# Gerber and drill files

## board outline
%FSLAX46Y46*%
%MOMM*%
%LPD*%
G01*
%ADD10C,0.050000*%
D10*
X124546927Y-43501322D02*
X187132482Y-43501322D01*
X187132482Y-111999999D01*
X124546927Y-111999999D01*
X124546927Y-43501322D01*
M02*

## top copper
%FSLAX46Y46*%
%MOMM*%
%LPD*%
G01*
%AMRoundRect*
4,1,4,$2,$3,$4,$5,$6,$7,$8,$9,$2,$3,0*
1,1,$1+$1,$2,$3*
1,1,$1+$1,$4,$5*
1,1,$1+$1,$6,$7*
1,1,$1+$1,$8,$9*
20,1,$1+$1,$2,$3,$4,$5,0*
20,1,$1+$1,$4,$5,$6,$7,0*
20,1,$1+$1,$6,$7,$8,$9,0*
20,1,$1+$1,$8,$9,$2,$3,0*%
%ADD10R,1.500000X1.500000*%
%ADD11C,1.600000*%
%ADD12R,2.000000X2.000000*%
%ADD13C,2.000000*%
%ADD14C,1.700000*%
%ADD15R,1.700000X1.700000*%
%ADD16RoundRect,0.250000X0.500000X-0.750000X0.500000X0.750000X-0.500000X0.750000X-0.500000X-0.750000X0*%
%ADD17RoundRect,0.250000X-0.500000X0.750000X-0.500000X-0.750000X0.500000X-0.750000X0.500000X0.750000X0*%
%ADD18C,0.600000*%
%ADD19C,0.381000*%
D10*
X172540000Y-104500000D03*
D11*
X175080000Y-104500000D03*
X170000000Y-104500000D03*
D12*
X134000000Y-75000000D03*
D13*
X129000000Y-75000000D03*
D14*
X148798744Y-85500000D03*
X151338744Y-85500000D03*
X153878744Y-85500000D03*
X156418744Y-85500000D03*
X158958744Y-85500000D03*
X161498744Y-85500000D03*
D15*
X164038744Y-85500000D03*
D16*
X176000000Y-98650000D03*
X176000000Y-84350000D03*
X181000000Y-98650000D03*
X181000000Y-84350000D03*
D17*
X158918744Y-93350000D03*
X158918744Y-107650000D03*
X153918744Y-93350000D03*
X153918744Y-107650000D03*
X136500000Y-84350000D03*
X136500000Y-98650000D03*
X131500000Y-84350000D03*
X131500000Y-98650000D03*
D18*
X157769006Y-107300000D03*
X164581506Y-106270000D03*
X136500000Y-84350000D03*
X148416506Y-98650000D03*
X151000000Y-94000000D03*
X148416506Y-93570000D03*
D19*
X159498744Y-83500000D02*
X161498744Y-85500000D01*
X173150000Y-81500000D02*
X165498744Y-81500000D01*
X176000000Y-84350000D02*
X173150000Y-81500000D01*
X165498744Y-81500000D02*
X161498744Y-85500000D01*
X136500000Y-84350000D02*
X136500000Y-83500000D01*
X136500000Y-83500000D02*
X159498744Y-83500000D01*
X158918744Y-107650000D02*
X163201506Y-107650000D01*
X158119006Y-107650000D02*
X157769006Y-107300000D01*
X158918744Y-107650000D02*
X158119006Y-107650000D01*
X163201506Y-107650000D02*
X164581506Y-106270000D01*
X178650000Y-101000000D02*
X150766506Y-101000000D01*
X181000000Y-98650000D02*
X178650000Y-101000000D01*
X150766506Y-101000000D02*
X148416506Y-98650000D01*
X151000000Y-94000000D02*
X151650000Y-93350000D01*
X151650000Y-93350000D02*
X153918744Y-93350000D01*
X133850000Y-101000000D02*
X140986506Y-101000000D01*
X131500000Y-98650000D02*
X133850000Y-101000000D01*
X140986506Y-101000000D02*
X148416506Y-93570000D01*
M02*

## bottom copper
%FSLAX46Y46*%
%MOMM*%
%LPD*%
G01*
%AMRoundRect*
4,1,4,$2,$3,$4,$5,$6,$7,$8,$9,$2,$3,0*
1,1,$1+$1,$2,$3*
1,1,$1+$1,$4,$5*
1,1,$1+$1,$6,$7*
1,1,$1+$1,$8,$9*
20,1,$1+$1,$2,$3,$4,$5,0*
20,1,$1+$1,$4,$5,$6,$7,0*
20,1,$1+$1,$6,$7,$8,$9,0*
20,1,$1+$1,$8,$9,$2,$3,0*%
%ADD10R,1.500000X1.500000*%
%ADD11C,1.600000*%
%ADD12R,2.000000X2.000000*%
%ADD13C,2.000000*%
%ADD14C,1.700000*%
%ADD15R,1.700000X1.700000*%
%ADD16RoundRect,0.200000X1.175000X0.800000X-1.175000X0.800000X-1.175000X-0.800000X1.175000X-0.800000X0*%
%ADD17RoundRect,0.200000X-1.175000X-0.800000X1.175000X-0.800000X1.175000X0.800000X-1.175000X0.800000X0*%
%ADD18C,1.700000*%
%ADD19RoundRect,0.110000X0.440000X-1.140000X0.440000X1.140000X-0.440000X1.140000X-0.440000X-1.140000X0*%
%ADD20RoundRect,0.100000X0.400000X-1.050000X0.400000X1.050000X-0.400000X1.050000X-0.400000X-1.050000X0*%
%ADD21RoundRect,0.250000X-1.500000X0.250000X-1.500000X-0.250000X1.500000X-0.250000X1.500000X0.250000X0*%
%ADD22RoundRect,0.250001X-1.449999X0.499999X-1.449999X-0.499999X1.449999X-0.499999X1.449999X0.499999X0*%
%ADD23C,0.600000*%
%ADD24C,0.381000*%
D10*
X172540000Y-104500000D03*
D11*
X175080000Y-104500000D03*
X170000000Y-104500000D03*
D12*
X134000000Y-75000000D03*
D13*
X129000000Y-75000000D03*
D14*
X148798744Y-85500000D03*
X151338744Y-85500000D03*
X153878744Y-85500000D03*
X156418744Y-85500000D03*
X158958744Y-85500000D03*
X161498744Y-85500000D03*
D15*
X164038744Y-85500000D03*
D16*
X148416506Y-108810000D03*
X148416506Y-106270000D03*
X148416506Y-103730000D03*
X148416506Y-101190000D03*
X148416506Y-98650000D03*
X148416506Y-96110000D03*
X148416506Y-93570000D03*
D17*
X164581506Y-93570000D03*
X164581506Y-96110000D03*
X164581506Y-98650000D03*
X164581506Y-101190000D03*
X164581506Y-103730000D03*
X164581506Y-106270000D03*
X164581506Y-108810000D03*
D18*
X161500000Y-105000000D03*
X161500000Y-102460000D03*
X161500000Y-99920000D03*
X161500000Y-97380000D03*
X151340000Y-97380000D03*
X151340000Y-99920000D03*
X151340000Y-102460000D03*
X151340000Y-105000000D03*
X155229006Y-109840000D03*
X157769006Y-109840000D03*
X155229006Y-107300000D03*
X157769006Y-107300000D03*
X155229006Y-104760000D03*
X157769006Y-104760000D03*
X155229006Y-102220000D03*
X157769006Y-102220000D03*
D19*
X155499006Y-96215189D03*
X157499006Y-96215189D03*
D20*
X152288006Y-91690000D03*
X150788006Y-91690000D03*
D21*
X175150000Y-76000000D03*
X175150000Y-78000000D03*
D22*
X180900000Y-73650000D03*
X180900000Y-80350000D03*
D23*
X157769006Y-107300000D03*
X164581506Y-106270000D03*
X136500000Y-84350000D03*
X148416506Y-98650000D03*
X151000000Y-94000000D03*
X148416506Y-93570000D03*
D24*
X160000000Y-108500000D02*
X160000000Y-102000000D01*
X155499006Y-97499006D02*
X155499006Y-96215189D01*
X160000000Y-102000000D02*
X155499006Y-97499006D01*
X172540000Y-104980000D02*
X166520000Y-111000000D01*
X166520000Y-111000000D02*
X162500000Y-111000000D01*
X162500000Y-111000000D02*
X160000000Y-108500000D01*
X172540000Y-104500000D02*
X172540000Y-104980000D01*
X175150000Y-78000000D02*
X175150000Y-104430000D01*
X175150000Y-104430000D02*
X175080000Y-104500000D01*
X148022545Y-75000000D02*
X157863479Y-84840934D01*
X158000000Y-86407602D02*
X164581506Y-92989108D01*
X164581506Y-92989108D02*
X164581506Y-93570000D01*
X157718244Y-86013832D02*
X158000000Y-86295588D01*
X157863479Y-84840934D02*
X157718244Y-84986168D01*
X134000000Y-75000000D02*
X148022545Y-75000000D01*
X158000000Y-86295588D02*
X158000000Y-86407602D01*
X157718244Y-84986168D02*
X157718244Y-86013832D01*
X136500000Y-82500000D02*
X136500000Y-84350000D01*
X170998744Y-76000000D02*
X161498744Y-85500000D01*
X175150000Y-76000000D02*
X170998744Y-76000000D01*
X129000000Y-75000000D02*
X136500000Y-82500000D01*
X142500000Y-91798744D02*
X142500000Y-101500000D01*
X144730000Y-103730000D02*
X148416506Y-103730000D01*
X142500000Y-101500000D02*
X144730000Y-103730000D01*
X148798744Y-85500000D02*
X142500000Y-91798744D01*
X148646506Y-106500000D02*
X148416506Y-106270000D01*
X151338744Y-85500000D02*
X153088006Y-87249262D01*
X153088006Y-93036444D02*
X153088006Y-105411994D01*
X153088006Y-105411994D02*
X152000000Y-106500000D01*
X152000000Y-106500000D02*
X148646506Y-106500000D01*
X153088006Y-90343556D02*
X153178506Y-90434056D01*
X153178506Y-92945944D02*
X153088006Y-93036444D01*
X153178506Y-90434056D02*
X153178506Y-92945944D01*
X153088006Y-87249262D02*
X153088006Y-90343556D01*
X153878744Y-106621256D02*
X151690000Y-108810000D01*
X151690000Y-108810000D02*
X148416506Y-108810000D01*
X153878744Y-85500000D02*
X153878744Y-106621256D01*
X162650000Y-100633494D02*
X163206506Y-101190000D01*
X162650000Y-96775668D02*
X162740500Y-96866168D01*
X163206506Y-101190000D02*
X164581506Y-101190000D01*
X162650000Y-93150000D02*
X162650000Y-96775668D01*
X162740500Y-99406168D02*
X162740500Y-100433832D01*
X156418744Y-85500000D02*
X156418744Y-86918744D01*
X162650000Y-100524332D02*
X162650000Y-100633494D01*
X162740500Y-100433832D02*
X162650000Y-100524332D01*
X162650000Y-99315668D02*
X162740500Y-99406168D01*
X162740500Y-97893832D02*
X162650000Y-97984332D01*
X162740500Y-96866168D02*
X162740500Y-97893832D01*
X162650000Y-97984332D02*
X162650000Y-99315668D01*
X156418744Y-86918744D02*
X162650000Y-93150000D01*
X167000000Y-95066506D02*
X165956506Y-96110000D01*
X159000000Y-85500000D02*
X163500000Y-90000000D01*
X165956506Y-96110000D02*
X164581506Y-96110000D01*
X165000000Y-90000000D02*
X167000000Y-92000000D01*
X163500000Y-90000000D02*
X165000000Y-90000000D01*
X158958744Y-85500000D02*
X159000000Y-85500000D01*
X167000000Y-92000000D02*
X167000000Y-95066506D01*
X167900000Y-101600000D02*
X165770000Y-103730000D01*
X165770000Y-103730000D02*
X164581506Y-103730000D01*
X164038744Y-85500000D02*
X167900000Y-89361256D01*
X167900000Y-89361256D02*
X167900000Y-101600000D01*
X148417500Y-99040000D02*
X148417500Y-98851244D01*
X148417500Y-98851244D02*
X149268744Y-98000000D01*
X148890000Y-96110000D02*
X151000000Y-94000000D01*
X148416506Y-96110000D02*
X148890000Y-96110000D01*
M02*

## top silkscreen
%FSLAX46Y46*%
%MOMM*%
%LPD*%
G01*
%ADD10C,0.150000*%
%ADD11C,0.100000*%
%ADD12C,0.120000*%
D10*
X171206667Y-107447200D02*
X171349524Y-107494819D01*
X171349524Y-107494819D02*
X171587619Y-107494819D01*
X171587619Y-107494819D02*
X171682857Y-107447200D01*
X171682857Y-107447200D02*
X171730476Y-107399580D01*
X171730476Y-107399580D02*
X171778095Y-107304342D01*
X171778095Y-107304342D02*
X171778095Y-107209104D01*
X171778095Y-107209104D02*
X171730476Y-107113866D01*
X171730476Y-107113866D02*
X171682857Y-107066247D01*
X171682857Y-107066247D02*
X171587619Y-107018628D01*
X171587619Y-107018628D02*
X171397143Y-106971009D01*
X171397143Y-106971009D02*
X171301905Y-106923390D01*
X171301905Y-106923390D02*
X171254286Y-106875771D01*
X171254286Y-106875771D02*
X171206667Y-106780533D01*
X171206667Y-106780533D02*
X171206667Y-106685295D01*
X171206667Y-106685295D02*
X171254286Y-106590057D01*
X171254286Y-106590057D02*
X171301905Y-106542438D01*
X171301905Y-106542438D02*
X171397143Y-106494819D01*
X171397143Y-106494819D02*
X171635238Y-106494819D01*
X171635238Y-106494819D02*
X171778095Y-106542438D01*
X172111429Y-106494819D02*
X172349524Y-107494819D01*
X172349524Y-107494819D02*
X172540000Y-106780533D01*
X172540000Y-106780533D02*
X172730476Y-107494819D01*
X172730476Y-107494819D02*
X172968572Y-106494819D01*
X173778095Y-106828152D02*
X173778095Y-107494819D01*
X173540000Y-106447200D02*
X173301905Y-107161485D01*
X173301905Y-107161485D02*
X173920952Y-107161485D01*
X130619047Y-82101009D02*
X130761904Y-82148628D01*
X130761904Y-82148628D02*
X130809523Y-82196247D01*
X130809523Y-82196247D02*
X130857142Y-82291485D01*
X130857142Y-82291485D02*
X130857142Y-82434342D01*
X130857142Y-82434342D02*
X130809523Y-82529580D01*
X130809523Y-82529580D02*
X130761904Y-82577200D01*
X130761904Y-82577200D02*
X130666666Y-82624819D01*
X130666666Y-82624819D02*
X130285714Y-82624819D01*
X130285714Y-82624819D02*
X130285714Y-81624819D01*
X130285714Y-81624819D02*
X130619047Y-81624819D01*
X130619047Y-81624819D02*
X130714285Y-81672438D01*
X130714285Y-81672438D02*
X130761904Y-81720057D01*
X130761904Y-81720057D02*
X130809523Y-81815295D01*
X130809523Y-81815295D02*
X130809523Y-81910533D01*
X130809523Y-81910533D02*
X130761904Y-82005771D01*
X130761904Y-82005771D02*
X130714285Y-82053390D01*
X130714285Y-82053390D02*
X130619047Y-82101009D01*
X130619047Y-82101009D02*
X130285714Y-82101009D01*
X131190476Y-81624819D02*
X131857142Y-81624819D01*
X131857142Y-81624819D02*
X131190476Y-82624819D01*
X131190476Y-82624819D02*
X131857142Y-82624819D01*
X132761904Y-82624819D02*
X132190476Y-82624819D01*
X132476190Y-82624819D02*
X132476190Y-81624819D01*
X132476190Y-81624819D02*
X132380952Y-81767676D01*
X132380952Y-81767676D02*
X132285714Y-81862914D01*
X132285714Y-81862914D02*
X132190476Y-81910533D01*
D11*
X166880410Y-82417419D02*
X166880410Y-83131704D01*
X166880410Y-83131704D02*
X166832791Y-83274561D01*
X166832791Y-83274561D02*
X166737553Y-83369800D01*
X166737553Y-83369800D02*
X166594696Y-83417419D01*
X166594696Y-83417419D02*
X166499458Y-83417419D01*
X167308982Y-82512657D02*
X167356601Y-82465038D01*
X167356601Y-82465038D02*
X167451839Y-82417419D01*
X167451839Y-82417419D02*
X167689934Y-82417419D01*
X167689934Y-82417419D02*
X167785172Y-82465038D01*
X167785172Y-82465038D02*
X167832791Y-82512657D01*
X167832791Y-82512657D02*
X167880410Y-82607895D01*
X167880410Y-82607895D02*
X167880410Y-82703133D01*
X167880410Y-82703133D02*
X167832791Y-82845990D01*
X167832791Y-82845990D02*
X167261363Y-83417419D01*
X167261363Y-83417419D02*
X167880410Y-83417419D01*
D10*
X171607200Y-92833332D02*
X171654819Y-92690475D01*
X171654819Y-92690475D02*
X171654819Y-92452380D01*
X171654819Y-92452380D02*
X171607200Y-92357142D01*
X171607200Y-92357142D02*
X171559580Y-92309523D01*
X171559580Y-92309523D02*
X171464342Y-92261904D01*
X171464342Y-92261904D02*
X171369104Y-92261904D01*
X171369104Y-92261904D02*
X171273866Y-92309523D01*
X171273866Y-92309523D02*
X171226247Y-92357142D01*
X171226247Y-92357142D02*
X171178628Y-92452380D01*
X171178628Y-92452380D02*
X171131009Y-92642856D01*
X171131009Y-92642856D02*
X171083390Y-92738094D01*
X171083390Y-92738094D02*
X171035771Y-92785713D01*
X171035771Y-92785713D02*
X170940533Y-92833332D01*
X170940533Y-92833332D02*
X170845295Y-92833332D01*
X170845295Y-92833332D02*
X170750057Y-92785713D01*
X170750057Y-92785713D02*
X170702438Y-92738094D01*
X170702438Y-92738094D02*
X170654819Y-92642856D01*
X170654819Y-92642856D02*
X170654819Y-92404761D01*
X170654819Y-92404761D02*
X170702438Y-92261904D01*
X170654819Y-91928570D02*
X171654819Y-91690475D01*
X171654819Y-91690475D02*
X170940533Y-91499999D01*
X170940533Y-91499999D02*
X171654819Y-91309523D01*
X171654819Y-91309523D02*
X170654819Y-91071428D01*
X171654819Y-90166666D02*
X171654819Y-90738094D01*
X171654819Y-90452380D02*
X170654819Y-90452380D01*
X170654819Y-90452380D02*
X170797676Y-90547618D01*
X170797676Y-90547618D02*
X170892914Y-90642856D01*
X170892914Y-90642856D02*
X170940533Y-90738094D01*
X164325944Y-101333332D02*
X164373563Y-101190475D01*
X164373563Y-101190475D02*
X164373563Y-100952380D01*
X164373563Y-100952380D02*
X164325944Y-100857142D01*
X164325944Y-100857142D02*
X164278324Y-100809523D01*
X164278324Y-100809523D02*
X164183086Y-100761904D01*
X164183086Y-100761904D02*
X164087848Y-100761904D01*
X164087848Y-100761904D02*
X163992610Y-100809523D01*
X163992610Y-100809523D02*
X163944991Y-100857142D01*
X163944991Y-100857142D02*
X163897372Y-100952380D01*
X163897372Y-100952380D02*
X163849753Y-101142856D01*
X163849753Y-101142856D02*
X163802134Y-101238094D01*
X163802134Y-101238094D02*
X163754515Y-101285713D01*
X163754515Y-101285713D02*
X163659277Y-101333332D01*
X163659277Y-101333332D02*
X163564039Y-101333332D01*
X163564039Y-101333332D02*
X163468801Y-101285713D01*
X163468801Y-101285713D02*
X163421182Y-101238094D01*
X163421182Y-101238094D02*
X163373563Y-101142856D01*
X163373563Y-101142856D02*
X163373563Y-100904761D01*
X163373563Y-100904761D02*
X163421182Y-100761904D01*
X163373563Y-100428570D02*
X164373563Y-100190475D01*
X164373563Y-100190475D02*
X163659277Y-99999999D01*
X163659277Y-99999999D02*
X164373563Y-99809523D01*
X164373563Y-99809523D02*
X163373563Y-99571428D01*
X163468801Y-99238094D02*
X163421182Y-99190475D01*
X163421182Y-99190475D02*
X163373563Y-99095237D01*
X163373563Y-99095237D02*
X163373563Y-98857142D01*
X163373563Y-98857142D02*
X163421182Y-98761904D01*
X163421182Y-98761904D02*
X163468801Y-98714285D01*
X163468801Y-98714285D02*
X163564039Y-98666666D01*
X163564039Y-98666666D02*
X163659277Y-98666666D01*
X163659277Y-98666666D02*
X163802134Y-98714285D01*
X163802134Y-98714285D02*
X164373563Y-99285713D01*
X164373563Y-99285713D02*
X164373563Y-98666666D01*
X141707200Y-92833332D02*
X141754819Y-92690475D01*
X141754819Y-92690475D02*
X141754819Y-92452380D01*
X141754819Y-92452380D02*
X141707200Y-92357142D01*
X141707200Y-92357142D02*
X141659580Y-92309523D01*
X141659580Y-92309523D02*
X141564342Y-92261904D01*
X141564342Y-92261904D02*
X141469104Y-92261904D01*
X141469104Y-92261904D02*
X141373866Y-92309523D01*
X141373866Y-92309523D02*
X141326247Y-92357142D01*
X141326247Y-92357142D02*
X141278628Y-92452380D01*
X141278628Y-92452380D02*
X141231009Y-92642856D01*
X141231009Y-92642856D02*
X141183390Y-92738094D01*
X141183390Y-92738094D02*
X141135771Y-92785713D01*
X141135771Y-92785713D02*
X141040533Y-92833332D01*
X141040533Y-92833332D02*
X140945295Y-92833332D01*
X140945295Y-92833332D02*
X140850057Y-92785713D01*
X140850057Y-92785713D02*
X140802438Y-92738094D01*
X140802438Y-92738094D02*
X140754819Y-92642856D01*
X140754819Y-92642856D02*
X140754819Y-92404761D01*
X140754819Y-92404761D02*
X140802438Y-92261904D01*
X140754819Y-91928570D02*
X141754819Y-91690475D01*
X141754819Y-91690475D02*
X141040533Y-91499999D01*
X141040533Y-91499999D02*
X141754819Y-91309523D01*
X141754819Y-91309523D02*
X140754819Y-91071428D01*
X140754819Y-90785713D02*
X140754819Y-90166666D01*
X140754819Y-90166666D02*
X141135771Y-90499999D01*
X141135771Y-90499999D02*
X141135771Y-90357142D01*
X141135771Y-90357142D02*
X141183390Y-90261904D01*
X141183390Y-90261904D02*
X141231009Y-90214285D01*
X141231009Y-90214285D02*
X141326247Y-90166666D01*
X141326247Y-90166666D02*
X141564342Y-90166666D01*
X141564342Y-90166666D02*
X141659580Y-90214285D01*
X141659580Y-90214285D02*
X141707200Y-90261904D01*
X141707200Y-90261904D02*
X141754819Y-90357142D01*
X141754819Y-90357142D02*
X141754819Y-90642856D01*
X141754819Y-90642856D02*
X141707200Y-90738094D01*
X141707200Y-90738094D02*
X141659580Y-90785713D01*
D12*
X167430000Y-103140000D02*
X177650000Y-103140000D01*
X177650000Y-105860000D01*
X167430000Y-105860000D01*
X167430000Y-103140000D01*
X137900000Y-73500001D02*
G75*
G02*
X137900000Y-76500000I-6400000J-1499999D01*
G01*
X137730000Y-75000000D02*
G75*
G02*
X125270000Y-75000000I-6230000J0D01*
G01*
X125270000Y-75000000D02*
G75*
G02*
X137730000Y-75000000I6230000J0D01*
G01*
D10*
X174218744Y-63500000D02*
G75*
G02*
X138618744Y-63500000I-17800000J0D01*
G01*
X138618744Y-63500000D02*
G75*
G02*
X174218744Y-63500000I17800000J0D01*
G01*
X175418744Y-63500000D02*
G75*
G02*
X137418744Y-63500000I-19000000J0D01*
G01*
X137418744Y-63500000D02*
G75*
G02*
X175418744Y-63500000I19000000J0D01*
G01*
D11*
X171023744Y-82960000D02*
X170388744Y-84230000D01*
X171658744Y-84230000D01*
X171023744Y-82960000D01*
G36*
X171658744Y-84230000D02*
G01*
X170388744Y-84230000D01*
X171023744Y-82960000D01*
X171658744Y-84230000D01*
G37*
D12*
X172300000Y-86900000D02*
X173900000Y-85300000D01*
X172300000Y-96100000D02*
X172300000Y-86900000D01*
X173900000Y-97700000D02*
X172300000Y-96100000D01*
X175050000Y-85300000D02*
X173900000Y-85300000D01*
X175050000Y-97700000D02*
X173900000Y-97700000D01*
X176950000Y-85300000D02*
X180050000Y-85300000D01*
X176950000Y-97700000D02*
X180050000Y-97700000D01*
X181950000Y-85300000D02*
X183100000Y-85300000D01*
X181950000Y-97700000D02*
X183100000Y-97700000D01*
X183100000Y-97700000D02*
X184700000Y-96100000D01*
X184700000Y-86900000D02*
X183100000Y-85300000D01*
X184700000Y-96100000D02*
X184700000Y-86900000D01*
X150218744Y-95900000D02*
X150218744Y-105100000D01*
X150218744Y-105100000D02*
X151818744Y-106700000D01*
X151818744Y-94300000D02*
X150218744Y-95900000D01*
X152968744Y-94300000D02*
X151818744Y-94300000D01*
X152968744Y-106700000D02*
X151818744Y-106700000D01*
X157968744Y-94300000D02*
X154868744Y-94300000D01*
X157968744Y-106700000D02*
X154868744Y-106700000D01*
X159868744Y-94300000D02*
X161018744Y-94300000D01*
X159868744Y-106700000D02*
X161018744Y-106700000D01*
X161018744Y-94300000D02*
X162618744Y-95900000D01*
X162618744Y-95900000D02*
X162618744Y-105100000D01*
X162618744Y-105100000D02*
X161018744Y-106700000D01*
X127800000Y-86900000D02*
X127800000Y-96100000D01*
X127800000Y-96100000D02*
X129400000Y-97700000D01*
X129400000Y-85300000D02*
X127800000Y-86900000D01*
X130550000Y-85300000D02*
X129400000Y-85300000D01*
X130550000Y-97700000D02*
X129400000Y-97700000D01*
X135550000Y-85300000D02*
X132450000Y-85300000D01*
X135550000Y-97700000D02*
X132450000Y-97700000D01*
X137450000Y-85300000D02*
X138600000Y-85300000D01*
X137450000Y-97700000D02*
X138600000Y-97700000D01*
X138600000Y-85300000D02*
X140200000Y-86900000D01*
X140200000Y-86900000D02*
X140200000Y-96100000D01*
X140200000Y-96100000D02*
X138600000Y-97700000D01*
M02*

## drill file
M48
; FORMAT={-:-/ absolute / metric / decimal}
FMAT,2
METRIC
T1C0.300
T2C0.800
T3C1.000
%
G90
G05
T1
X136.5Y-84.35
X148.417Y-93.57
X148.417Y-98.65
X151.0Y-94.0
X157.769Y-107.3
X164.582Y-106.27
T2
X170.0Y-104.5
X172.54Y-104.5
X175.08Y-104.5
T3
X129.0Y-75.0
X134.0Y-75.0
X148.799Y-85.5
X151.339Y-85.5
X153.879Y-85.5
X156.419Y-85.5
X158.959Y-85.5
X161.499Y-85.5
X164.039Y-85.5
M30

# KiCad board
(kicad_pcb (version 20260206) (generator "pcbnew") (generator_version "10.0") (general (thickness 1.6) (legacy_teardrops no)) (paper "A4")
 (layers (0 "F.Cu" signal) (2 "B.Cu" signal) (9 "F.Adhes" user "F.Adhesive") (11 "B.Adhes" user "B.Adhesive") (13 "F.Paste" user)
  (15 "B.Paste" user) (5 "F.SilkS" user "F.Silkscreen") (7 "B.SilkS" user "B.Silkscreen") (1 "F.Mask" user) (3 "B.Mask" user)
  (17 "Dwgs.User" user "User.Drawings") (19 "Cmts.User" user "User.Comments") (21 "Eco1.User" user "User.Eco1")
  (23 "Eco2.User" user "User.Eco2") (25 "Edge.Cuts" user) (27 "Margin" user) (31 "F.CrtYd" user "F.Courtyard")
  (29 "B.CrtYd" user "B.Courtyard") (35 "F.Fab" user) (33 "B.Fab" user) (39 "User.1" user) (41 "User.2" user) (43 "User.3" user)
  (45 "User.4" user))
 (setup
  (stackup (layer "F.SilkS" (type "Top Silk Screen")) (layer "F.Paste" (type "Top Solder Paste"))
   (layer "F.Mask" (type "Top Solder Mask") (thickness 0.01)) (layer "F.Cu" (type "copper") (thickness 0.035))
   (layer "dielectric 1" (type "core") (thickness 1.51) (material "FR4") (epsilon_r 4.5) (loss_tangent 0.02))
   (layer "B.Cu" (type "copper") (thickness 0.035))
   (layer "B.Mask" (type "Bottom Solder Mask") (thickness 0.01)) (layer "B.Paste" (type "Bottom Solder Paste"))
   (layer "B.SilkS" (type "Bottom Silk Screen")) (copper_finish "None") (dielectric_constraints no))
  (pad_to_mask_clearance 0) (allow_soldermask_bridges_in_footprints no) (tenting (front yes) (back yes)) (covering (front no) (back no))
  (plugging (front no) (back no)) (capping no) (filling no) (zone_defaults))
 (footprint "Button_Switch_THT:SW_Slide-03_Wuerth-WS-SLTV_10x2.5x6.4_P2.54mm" (layer "F.Cu") (at 172.54 104.5 180)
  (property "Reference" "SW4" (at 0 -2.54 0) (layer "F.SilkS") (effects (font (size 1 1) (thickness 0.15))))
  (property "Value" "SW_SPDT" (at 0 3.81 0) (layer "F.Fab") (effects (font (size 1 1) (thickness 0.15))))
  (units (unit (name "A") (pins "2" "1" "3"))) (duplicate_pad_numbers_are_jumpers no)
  (fp_rect (start -5.11 -1.36) (end 5.11 1.36) (stroke (width 0.12) (type default)) (fill no) (layer "F.SilkS"))
  (pad "1" thru_hole rect (at 0 0 180) (size 1.5 1.5) (drill 0.8) (layers "*.Cu" "*.Mask") (remove_unused_layers no) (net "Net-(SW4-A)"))
  (pad "2" thru_hole circle (at -2.54 0 180) (size 1.6 1.6) (drill 0.8) (layers "*.Cu" "*.Mask") (remove_unused_layers no)
   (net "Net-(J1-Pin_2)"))
  (pad "3" thru_hole circle (at 2.54 0 180) (size 1.6 1.6) (drill 0.8) (layers "*.Cu" "*.Mask") (remove_unused_layers no)
   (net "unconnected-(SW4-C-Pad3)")))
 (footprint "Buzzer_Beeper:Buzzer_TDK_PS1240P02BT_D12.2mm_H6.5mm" (layer "F.Cu") (at 134 75 180)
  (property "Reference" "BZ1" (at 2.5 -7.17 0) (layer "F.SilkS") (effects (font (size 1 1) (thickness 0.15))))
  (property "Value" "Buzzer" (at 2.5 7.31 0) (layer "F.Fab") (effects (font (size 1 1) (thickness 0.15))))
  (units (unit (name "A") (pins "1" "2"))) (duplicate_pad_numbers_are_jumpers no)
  (fp_arc (start -3.9 1.499999) (mid -4.073431 0) (end -3.9 -1.5) (stroke (width 0.12) (type solid)) (layer "F.SilkS"))
  (fp_circle (center 2.5 0) (end 8.73 0) (stroke (width 0.12) (type solid)) (fill no) (layer "F.SilkS"))
  (pad "1" thru_hole rect (at 0 0 180) (size 2 2) (drill 1) (layers "*.Cu" "*.Mask") (remove_unused_layers no) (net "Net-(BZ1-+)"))
  (pad "2" thru_hole circle (at 5 0 180) (size 2 2) (drill 1) (layers "*.Cu" "*.Mask") (remove_unused_layers no) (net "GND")))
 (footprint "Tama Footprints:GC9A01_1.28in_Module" (layer "F.Cu") (at 164.038744 85.5)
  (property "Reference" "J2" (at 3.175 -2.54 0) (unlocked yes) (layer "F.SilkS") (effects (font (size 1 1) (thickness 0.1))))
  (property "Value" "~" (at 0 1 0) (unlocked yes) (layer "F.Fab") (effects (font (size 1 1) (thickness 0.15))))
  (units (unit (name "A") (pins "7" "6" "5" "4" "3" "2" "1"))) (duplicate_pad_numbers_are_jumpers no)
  (fp_circle (center -7.62 -22) (end 10.18 -22) (stroke (width 0.15) (type solid)) (fill no) (layer "F.SilkS"))
  (fp_circle (center -7.62 -22) (end 11.38 -22) (stroke (width 0.15) (type solid)) (fill no) (layer "F.SilkS"))
  (fp_poly (pts (xy 6.985 -2.54) (xy 6.35 -1.27) (xy 7.62 -1.27)) (stroke (width 0.1) (type solid)) (fill yes) (layer "F.SilkS"))
  (pad "1" thru_hole circle (at -15.24 0) (size 1.7 1.7) (drill 1) (layers "*.Cu" "*.Mask") (remove_unused_layers no) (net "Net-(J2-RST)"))
  (pad "2" thru_hole circle (at -12.7 0) (size 1.7 1.7) (drill 1) (layers "*.Cu" "*.Mask") (remove_unused_layers no) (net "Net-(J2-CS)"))
  (pad "3" thru_hole circle (at -10.16 0) (size 1.7 1.7) (drill 1) (layers "*.Cu" "*.Mask") (remove_unused_layers no) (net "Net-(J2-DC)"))
  (pad "4" thru_hole circle (at -7.62 0) (size 1.7 1.7) (drill 1) (layers "*.Cu" "*.Mask") (remove_unused_layers no) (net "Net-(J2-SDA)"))
  (pad "5" thru_hole circle (at -5.08 0) (size 1.7 1.7) (drill 1) (layers "*.Cu" "*.Mask") (remove_unused_layers no) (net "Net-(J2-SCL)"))
  (pad "6" thru_hole circle (at -2.54 0) (size 1.7 1.7) (drill 1) (layers "*.Cu" "*.Mask") (remove_unused_layers no) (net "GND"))
  (pad "7" thru_hole rect (at 0 0) (size 1.7 1.7) (drill 1) (layers "*.Cu" "*.Mask") (remove_unused_layers no) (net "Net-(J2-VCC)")))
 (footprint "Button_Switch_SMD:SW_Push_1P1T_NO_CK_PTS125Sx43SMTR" (layer "F.Cu") (at 178.5 91.5 90)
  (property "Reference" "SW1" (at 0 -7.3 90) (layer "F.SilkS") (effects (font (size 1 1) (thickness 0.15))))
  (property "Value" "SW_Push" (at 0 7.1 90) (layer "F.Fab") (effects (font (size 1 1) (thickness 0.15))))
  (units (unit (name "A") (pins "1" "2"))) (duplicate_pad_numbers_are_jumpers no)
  (fp_line (start 4.6 -6.2) (end 6.2 -4.6) (stroke (width 0.12) (type solid)) (layer "F.SilkS"))
  (fp_line (start -4.6 -6.2) (end 4.6 -6.2) (stroke (width 0.12) (type solid)) (layer "F.SilkS"))
  (fp_line (start -6.2 -4.6) (end -4.6 -6.2) (stroke (width 0.12) (type solid)) (layer "F.SilkS"))
  (fp_line (start 6.2 -3.45) (end 6.2 -4.6) (stroke (width 0.12) (type solid)) (layer "F.SilkS"))
  (fp_line (start -6.2 -3.45) (end -6.2 -4.6) (stroke (width 0.12) (type solid)) (layer "F.SilkS"))
  (fp_line (start 6.2 -1.55) (end 6.2 1.55) (stroke (width 0.12) (type solid)) (layer "F.SilkS"))
  (fp_line (start -6.2 -1.55) (end -6.2 1.55) (stroke (width 0.12) (type solid)) (layer "F.SilkS"))
  (fp_line (start 6.2 3.45) (end 6.2 4.6) (stroke (width 0.12) (type solid)) (layer "F.SilkS"))
  (fp_line (start -6.2 3.45) (end -6.2 4.6) (stroke (width 0.12) (type solid)) (layer "F.SilkS"))
  (fp_line (start -6.2 4.6) (end -4.6 6.2) (stroke (width 0.12) (type solid)) (layer "F.SilkS"))
  (fp_line (start 4.6 6.2) (end 6.2 4.6) (stroke (width 0.12) (type solid)) (layer "F.SilkS"))
  (fp_line (start -4.6 6.2) (end 4.6 6.2) (stroke (width 0.12) (type solid)) (layer "F.SilkS"))
  (pad "1" smd roundrect (at -7.15 -2.5 90) (size 2 1.5) (layers "F.Cu" "F.Mask" "F.Paste") (roundrect_rratio 0.1666666667))
  (pad "1" smd roundrect (at 7.15 -2.5 90) (size 2 1.5) (layers "F.Cu" "F.Mask" "F.Paste") (roundrect_rratio 0.1666666667) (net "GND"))
  (pad "2" smd roundrect (at -7.15 2.5 90) (size 2 1.5) (layers "F.Cu" "F.Mask" "F.Paste") (roundrect_rratio 0.1666666667)
   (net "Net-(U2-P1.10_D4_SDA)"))
  (pad "2" smd roundrect (at 7.15 2.5 90) (size 2 1.5) (layers "F.Cu" "F.Mask" "F.Paste") (roundrect_rratio 0.1666666667)))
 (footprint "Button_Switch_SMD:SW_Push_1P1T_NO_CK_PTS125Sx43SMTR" (layer "F.Cu") (at 156.418744 100.5 -90)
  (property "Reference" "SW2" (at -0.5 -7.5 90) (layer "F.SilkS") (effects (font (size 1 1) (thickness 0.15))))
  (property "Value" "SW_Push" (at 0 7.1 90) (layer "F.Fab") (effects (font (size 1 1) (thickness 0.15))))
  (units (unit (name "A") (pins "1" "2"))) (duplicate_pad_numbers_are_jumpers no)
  (fp_line (start -4.6 6.2) (end 4.6 6.2) (stroke (width 0.12) (type solid)) (layer "F.SilkS"))
  (fp_line (start 4.6 6.2) (end 6.2 4.6) (stroke (width 0.12) (type solid)) (layer "F.SilkS"))
  (fp_line (start -6.2 4.6) (end -4.6 6.2) (stroke (width 0.12) (type solid)) (layer "F.SilkS"))
  (fp_line (start -6.2 3.45) (end -6.2 4.6) (stroke (width 0.12) (type solid)) (layer "F.SilkS"))
  (fp_line (start 6.2 3.45) (end 6.2 4.6) (stroke (width 0.12) (type solid)) (layer "F.SilkS"))
  (fp_line (start -6.2 -1.55) (end -6.2 1.55) (stroke (width 0.12) (type solid)) (layer "F.SilkS"))
  (fp_line (start 6.2 -1.55) (end 6.2 1.55) (stroke (width 0.12) (type solid)) (layer "F.SilkS"))
  (fp_line (start -6.2 -3.45) (end -6.2 -4.6) (stroke (width 0.12) (type solid)) (layer "F.SilkS"))
  (fp_line (start 6.2 -3.45) (end 6.2 -4.6) (stroke (width 0.12) (type solid)) (layer "F.SilkS"))
  (fp_line (start -6.2 -4.6) (end -4.6 -6.2) (stroke (width 0.12) (type solid)) (layer "F.SilkS"))
  (fp_line (start -4.6 -6.2) (end 4.6 -6.2) (stroke (width 0.12) (type solid)) (layer "F.SilkS"))
  (fp_line (start 4.6 -6.2) (end 6.2 -4.6) (stroke (width 0.12) (type solid)) (layer "F.SilkS"))
  (pad "1" smd roundrect (at -7.15 -2.5 270) (size 2 1.5) (layers "F.Cu" "F.Mask" "F.Paste") (roundrect_rratio 0.1666666667))
  (pad "1" smd roundrect (at 7.15 -2.5 270) (size 2 1.5) (layers "F.Cu" "F.Mask" "F.Paste") (roundrect_rratio 0.1666666667) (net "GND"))
  (pad "2" smd roundrect (at -7.15 2.5 270) (size 2 1.5) (layers "F.Cu" "F.Mask" "F.Paste") (roundrect_rratio 0.1666666667)
   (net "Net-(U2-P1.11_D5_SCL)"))
  (pad "2" smd roundrect (at 7.15 2.5 270) (size 2 1.5) (layers "F.Cu" "F.Mask" "F.Paste") (roundrect_rratio 0.1666666667)))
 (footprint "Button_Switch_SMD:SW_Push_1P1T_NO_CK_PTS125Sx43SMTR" (layer "F.Cu") (at 134 91.5 -90)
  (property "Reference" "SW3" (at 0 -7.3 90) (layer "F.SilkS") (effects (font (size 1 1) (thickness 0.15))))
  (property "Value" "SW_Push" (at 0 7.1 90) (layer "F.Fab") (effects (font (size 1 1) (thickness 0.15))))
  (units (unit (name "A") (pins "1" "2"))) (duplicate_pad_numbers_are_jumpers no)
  (fp_line (start -4.6 6.2) (end 4.6 6.2) (stroke (width 0.12) (type solid)) (layer "F.SilkS"))
  (fp_line (start 4.6 6.2) (end 6.2 4.6) (stroke (width 0.12) (type solid)) (layer "F.SilkS"))
  (fp_line (start -6.2 4.6) (end -4.6 6.2) (stroke (width 0.12) (type solid)) (layer "F.SilkS"))
  (fp_line (start -6.2 3.45) (end -6.2 4.6) (stroke (width 0.12) (type solid)) (layer "F.SilkS"))
  (fp_line (start 6.2 3.45) (end 6.2 4.6) (stroke (width 0.12) (type solid)) (layer "F.SilkS"))
  (fp_line (start -6.2 -1.55) (end -6.2 1.55) (stroke (width 0.12) (type solid)) (layer "F.SilkS"))
  (fp_line (start 6.2 -1.55) (end 6.2 1.55) (stroke (width 0.12) (type solid)) (layer "F.SilkS"))
  (fp_line (start -6.2 -3.45) (end -6.2 -4.6) (stroke (width 0.12) (type solid)) (layer "F.SilkS"))
  (fp_line (start 6.2 -3.45) (end 6.2 -4.6) (stroke (width 0.12) (type solid)) (layer "F.SilkS"))
  (fp_line (start -6.2 -4.6) (end -4.6 -6.2) (stroke (width 0.12) (type solid)) (layer "F.SilkS"))
  (fp_line (start -4.6 -6.2) (end 4.6 -6.2) (stroke (width 0.12) (type solid)) (layer "F.SilkS"))
  (fp_line (start 4.6 -6.2) (end 6.2 -4.6) (stroke (width 0.12) (type solid)) (layer "F.SilkS"))
  (pad "1" smd roundrect (at -7.15 -2.5 270) (size 2 1.5) (layers "F.Cu" "F.Mask" "F.Paste") (roundrect_rratio 0.1666666667) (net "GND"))
  (pad "1" smd roundrect (at 7.15 -2.5 270) (size 2 1.5) (layers "F.Cu" "F.Mask" "F.Paste") (roundrect_rratio 0.1666666667))
  (pad "2" smd roundrect (at -7.15 2.5 270) (size 2 1.5) (layers "F.Cu" "F.Mask" "F.Paste") (roundrect_rratio 0.1666666667))
  (pad "2" smd roundrect (at 7.15 2.5 270) (size 2 1.5) (layers "F.Cu" "F.Mask" "F.Paste") (roundrect_rratio 0.1666666667)
   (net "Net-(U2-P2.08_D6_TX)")))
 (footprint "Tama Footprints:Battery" (layer "B.Cu") (at 156.418744 64.5 -90)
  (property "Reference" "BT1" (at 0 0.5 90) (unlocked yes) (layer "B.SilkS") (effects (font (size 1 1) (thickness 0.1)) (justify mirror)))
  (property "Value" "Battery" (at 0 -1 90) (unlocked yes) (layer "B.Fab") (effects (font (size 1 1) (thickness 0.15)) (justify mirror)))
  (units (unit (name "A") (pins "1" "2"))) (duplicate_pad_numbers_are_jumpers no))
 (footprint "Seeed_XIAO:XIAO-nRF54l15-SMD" (layer "B.Cu") (at 156.499006 101.19 -90)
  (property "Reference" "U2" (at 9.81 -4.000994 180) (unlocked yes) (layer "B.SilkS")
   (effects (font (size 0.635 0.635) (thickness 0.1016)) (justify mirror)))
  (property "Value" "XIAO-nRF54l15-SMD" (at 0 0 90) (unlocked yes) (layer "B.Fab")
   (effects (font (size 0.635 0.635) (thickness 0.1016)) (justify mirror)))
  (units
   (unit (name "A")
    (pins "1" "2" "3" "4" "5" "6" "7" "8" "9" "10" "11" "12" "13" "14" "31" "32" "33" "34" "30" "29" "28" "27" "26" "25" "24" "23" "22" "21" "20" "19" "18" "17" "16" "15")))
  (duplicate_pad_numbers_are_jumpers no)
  (pad "1" smd roundrect (at 7.62 8.0825 180) (size 2.75 2) (layers "B.Cu" "B.Mask" "B.Paste") (roundrect_rratio 0.1) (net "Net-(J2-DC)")
   (thermal_bridge_angle 45))
  (pad "2" smd roundrect (at 5.08 8.0825 180) (size 2.75 2) (layers "B.Cu" "B.Mask" "B.Paste") (roundrect_rratio 0.1) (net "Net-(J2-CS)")
   (thermal_bridge_angle 45))
  (pad "3" smd roundrect (at 2.54 8.0825 180) (size 2.75 2) (layers "B.Cu" "B.Mask" "B.Paste") (roundrect_rratio 0.1) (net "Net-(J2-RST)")
   (thermal_bridge_angle 45))
  (pad "4" smd roundrect (at 0 8.0825 180) (size 2.75 2) (layers "B.Cu" "B.Mask" "B.Paste") (roundrect_rratio 0.1)
   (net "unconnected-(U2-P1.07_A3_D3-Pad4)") (thermal_bridge_angle 45))
  (pad "5" smd roundrect (at -2.54 8.0825 180) (size 2.75 2) (layers "B.Cu" "B.Mask" "B.Paste") (roundrect_rratio 0.1)
   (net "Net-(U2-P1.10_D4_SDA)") (thermal_bridge_angle 45))
  (pad "6" smd roundrect (at -5.08 8.0825 180) (size 2.75 2) (layers "B.Cu" "B.Mask" "B.Paste") (roundrect_rratio 0.1)
   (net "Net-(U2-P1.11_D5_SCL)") (thermal_bridge_angle 45))
  (pad "7" smd roundrect (at -7.62 8.0825 180) (size 2.75 2) (layers "B.Cu" "B.Mask" "B.Paste") (roundrect_rratio 0.1)
   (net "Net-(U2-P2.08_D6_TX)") (thermal_bridge_angle 45))
  (pad "8" smd roundrect (at -7.62 -8.0825) (size 2.75 2) (layers "B.Cu" "B.Mask" "B.Paste") (roundrect_rratio 0.1) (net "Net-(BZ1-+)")
   (thermal_bridge_angle 45))
  (pad "9" smd roundrect (at -5.08 -8.0825) (size 2.75 2) (layers "B.Cu" "B.Mask" "B.Paste") (roundrect_rratio 0.1) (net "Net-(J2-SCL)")
   (thermal_bridge_angle 45))
  (pad "10" smd roundrect (at -2.54 -8.0825) (size 2.75 2) (layers "B.Cu" "B.Mask" "B.Paste") (roundrect_rratio 0.1)
   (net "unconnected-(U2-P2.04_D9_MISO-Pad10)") (thermal_bridge_angle 45))
  (pad "11" smd roundrect (at 0 -8.0825) (size 2.75 2) (layers "B.Cu" "B.Mask" "B.Paste") (roundrect_rratio 0.1) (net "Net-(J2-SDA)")
   (thermal_bridge_angle 45))
  (pad "12" smd roundrect (at 2.54 -8.0825) (size 2.75 2) (layers "B.Cu" "B.Mask" "B.Paste") (roundrect_rratio 0.1) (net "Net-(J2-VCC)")
   (thermal_bridge_angle 45))
  (pad "13" smd roundrect (at 5.08 -8.0825) (size 2.75 2) (layers "B.Cu" "B.Mask" "B.Paste") (roundrect_rratio 0.1) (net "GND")
   (thermal_bridge_angle 45))
  (pad "14" smd roundrect (at 7.62 -8.0825) (size 2.75 2) (layers "B.Cu" "B.Mask" "B.Paste") (roundrect_rratio 0.1)
   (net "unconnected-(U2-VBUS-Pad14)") (thermal_bridge_angle 45))
  (pad "15" smd circle (at 3.81 -5.000994 180) (size 1.7 1.7) (layers "B.Cu" "B.Mask" "B.Paste")
   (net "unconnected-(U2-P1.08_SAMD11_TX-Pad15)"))
  (pad "16" smd circle (at 1.27 -5.000994 180) (size 1.7 1.7) (layers "B.Cu" "B.Mask" "B.Paste")
   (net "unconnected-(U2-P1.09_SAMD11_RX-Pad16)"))
  (pad "17" smd circle (at -1.27 -5.000994 180) (size 1.7 1.7) (layers "B.Cu" "B.Mask" "B.Paste") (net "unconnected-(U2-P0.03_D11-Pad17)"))
  (pad "18" smd circle (at -3.81 -5.000994 180) (size 1.7 1.7) (layers "B.Cu" "B.Mask" "B.Paste") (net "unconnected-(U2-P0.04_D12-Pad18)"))
  (pad "19" smd circle (at -3.81 5.159006 180) (size 1.7 1.7) (layers "B.Cu" "B.Mask" "B.Paste") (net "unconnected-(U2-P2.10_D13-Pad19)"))
  (pad "20" smd circle (at -1.27 5.159006 180) (size 1.7 1.7) (layers "B.Cu" "B.Mask" "B.Paste") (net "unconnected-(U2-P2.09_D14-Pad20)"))
  (pad "21" smd circle (at 1.27 5.159006 180) (size 1.7 1.7) (layers "B.Cu" "B.Mask" "B.Paste") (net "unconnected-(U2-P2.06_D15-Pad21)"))
  (pad "22" smd circle (at 3.81 5.159006 180) (size 1.7 1.7) (layers "B.Cu" "B.Mask" "B.Paste") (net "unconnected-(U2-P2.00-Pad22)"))
  (pad "23" smd circle (at 8.65 1.27 180) (size 1.7 1.7) (layers "B.Cu" "B.Mask" "B.Paste") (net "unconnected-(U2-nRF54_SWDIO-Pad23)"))
  (pad "24" smd circle (at 8.65 -1.27 180) (size 1.7 1.7) (layers "B.Cu" "B.Mask" "B.Paste") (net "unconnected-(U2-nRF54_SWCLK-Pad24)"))
  (pad "25" smd circle (at 6.11 1.27 180) (size 1.7 1.7) (layers "B.Cu" "B.Mask" "B.Paste") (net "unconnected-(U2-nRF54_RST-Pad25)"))
  (pad "26" smd circle (at 6.11 -1.27 180) (size 1.7 1.7) (layers "B.Cu" "B.Mask" "B.Paste") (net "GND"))
  (pad "27" smd circle (at 3.57 1.27 180) (size 1.7 1.7) (layers "B.Cu" "B.Mask" "B.Paste") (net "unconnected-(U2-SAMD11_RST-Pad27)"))
  (pad "28" smd circle (at 3.57 -1.27 180) (size 1.7 1.7) (layers "B.Cu" "B.Mask" "B.Paste") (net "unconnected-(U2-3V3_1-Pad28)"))
  (pad "29" smd circle (at 1.03 1.27 180) (size 1.7 1.7) (layers "B.Cu" "B.Mask" "B.Paste") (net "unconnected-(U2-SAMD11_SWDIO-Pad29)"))
  (pad "30" smd circle (at 1.03 -1.27 180) (size 1.7 1.7) (layers "B.Cu" "B.Mask" "B.Paste") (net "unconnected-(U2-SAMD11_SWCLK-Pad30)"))
  (pad "31" smd roundrect (at -4.974811 1 90) (size 2.5 1.1) (layers "B.Cu" "B.Mask" "B.Paste") (roundrect_rratio 0.1) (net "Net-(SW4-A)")
   (thermal_bridge_angle 45))
  (pad "32" smd roundrect (at -4.974811 -1 90) (size 2.5 1.1) (layers "B.Cu" "B.Mask" "B.Paste") (roundrect_rratio 0.1)
   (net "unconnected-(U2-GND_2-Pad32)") (thermal_bridge_angle 45))
  (pad "33" smd roundrect (at -9.5 4.211 90) (size 2.3 1) (layers "B.Cu" "B.Mask" "B.Paste") (roundrect_rratio 0.1)
   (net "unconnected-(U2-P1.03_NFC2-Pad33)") (thermal_bridge_angle 45))
  (pad "34" smd roundrect (at -9.5 5.711 90) (size 2.3 1) (layers "B.Cu" "B.Mask" "B.Paste") (roundrect_rratio 0.1)
   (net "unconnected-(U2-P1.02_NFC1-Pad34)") (thermal_bridge_angle 45)))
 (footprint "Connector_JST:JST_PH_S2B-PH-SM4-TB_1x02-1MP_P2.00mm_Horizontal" (layer "B.Cu") (at 178 77 -90)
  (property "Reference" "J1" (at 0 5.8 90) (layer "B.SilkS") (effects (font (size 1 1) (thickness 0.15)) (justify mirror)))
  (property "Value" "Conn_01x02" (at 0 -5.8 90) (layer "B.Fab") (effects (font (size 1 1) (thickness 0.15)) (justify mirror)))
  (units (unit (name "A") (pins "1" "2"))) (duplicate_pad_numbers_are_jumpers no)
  (pad "1" smd roundrect (at -1 2.85 270) (size 1 3.5) (layers "B.Cu" "B.Mask" "B.Paste") (roundrect_rratio 0.25) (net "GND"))
  (pad "2" smd roundrect (at 1 2.85 270) (size 1 3.5) (layers "B.Cu" "B.Mask" "B.Paste") (roundrect_rratio 0.25) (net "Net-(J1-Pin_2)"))
  (pad "MP" smd roundrect (at -3.35 -2.9 270) (size 1.5 3.4) (layers "B.Cu" "B.Mask" "B.Paste") (roundrect_rratio 0.166667))
  (pad "MP" smd roundrect (at 3.35 -2.9 270) (size 1.5 3.4) (layers "B.Cu" "B.Mask" "B.Paste") (roundrect_rratio 0.166667)))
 (gr_rect (start 124.546927 43.501322) (end 187.132482 111.999999) (stroke (width 0.05) (type default)) (fill no) (layer "Edge.Cuts"))
 (segment (start 160 108.5) (end 160 102) (width 0.381) (layer "B.Cu") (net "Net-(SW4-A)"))
 (segment (start 155.499006 97.499006) (end 155.499006 96.215189) (width 0.381) (layer "B.Cu") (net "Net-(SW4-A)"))
 (segment (start 160 102) (end 155.499006 97.499006) (width 0.381) (layer "B.Cu") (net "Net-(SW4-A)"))
 (segment (start 172.54 104.98) (end 166.52 111) (width 0.381) (layer "B.Cu") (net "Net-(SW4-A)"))
 (segment (start 166.52 111) (end 162.5 111) (width 0.381) (layer "B.Cu") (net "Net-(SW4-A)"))
 (segment (start 162.5 111) (end 160 108.5) (width 0.381) (layer "B.Cu") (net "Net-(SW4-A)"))
 (segment (start 172.54 104.5) (end 172.54 104.98) (width 0.381) (layer "B.Cu") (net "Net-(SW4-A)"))
 (segment (start 175.15 78) (end 175.15 104.43) (width 0.381) (layer "B.Cu") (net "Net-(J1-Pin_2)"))
 (segment (start 175.15 104.43) (end 175.08 104.5) (width 0.381) (layer "B.Cu") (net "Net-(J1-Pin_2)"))
 (segment (start 148.022545 75) (end 157.863479 84.840934) (width 0.381) (layer "B.Cu") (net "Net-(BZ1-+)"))
 (segment (start 158 86.407602) (end 164.581506 92.989108) (width 0.381) (layer "B.Cu") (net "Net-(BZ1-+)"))
 (segment (start 164.581506 92.989108) (end 164.581506 93.57) (width 0.381) (layer "B.Cu") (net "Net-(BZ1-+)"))
 (segment (start 157.718244 86.013832) (end 158 86.295588) (width 0.381) (layer "B.Cu") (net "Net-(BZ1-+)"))
 (segment (start 157.863479 84.840934) (end 157.718244 84.986168) (width 0.381) (layer "B.Cu") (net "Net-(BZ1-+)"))
 (segment (start 134 75) (end 148.022545 75) (width 0.381) (layer "B.Cu") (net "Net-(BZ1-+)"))
 (segment (start 158 86.295588) (end 158 86.407602) (width 0.381) (layer "B.Cu") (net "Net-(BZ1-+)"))
 (segment (start 157.718244 84.986168) (end 157.718244 86.013832) (width 0.381) (layer "B.Cu") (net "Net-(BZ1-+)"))
 (segment (start 159.498744 83.5) (end 161.498744 85.5) (width 0.381) (layer "F.Cu") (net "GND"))
 (segment (start 173.15 81.5) (end 165.498744 81.5) (width 0.381) (layer "F.Cu") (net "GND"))
 (segment (start 176 84.35) (end 173.15 81.5) (width 0.381) (layer "F.Cu") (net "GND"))
 (segment (start 165.498744 81.5) (end 161.498744 85.5) (width 0.381) (layer "F.Cu") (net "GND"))
 (segment (start 136.5 84.35) (end 136.5 83.5) (width 0.381) (layer "F.Cu") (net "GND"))
 (segment (start 136.5 83.5) (end 159.498744 83.5) (width 0.381) (layer "F.Cu") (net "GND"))
 (segment (start 158.918744 107.65) (end 163.201506 107.65) (width 0.381) (layer "F.Cu") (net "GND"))
 (segment (start 158.119006 107.65) (end 157.769006 107.3) (width 0.381) (layer "F.Cu") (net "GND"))
 (segment (start 158.918744 107.65) (end 158.119006 107.65) (width 0.381) (layer "F.Cu") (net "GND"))
 (segment (start 163.201506 107.65) (end 164.581506 106.27) (width 0.381) (layer "F.Cu") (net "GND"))
 (via (at 157.769006 107.3) (size 0.6) (drill 0.3) (layers "F.Cu" "B.Cu") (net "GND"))
 (via (at 164.581506 106.27) (size 0.6) (drill 0.3) (layers "F.Cu" "B.Cu") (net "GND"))
 (via (at 136.5 84.35) (size 0.6) (drill 0.3) (layers "F.Cu" "B.Cu") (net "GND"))
 (segment (start 136.5 82.5) (end 136.5 84.35) (width 0.381) (layer "B.Cu") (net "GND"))
 (segment (start 170.998744 76) (end 161.498744 85.5) (width 0.381) (layer "B.Cu") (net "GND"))
 (segment (start 175.15 76) (end 170.998744 76) (width 0.381) (layer "B.Cu") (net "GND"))
 (segment (start 129 75) (end 136.5 82.5) (width 0.381) (layer "B.Cu") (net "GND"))
 (segment (start 142.5 91.798744) (end 142.5 101.5) (width 0.381) (layer "B.Cu") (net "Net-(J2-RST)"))
 (segment (start 144.73 103.73) (end 148.416506 103.73) (width 0.381) (layer "B.Cu") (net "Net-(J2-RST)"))
 (segment (start 142.5 101.5) (end 144.73 103.73) (width 0.381) (layer "B.Cu") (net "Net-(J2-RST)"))
 (segment (start 148.798744 85.5) (end 142.5 91.798744) (width 0.381) (layer "B.Cu") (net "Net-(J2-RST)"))
 (segment (start 148.646506 106.5) (end 148.416506 106.27) (width 0.381) (layer "B.Cu") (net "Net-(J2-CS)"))
 (segment (start 151.338744 85.5) (end 153.088006 87.249262) (width 0.381) (layer "B.Cu") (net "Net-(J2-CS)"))
 (segment (start 153.088006 93.036444) (end 153.088006 105.411994) (width 0.381) (layer "B.Cu") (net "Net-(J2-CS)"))
 (segment (start 153.088006 105.411994) (end 152 106.5) (width 0.381) (layer "B.Cu") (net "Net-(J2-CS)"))
 (segment (start 152 106.5) (end 148.646506 106.5) (width 0.381) (layer "B.Cu") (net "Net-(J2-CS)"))
 (segment (start 153.088006 90.343556) (end 153.178506 90.434056) (width 0.381) (layer "B.Cu") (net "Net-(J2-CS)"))
 (segment (start 153.178506 92.945944) (end 153.088006 93.036444) (width 0.381) (layer "B.Cu") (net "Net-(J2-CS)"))
 (segment (start 153.178506 90.434056) (end 153.178506 92.945944) (width 0.381) (layer "B.Cu") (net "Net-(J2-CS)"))
 (segment (start 153.088006 87.249262) (end 153.088006 90.343556) (width 0.381) (layer "B.Cu") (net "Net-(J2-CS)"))
 (segment (start 153.878744 106.621256) (end 151.69 108.81) (width 0.381) (layer "B.Cu") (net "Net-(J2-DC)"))
 (segment (start 151.69 108.81) (end 148.416506 108.81) (width 0.381) (layer "B.Cu") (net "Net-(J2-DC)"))
 (segment (start 153.878744 85.5) (end 153.878744 106.621256) (width 0.381) (layer "B.Cu") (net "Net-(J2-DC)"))
 (segment (start 162.65 100.633494) (end 163.206506 101.19) (width 0.381) (layer "B.Cu") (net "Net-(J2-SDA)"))
 (segment (start 162.65 96.775668) (end 162.7405 96.866168) (width 0.381) (layer "B.Cu") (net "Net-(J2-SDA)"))
 (segment (start 163.206506 101.19) (end 164.581506 101.19) (width 0.381) (layer "B.Cu") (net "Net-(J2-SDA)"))
 (segment (start 162.65 93.15) (end 162.65 96.775668) (width 0.381) (layer "B.Cu") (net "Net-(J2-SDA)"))
 (segment (start 162.7405 99.406168) (end 162.7405 100.433832) (width 0.381) (layer "B.Cu") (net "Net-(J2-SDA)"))
 (segment (start 156.418744 85.5) (end 156.418744 86.918744) (width 0.381) (layer "B.Cu") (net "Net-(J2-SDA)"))
 (segment (start 162.65 100.524332) (end 162.65 100.633494) (width 0.381) (layer "B.Cu") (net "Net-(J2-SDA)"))
 (segment (start 162.7405 100.433832) (end 162.65 100.524332) (width 0.381) (layer "B.Cu") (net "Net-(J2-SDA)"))
 (segment (start 162.65 99.315668) (end 162.7405 99.406168) (width 0.381) (layer "B.Cu") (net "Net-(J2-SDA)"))
 (segment (start 162.7405 97.893832) (end 162.65 97.984332) (width 0.381) (layer "B.Cu") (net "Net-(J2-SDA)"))
 (segment (start 162.7405 96.866168) (end 162.7405 97.893832) (width 0.381) (layer "B.Cu") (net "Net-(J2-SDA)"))
 (segment (start 162.65 97.984332) (end 162.65 99.315668) (width 0.381) (layer "B.Cu") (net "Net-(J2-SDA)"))
 (segment (start 156.418744 86.918744) (end 162.65 93.15) (width 0.381) (layer "B.Cu") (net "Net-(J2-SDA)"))
 (segment (start 167 95.066506) (end 165.956506 96.11) (width 0.381) (layer "B.Cu") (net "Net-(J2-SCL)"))
 (segment (start 159 85.5) (end 163.5 90) (width 0.381) (layer "B.Cu") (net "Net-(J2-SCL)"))
 (segment (start 165.956506 96.11) (end 164.581506 96.11) (width 0.381) (layer "B.Cu") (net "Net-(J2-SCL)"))
 (segment (start 165 90) (end 167 92) (width 0.381) (layer "B.Cu") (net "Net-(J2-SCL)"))
 (segment (start 163.5 90) (end 165 90) (width 0.381) (layer "B.Cu") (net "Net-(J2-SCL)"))
 (segment (start 158.958744 85.5) (end 159 85.5) (width 0.381) (layer "B.Cu") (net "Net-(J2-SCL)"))
 (segment (start 167 92) (end 167 95.066506) (width 0.381) (layer "B.Cu") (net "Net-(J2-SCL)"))
 (segment (start 167.9 101.6) (end 165.77 103.73) (width 0.381) (layer "B.Cu") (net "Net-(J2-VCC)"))
 (segment (start 165.77 103.73) (end 164.581506 103.73) (width 0.381) (layer "B.Cu") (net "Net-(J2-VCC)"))
 (segment (start 164.038744 85.5) (end 167.9 89.361256) (width 0.381) (layer "B.Cu") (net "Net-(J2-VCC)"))
 (segment (start 167.9 89.361256) (end 167.9 101.6) (width 0.381) (layer "B.Cu") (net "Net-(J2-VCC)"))
 (segment (start 178.65 101) (end 150.766506 101) (width 0.381) (layer "F.Cu") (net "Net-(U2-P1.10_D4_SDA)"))
 (segment (start 181 98.65) (end 178.65 101) (width 0.381) (layer "F.Cu") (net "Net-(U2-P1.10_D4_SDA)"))
 (segment (start 150.766506 101) (end 148.416506 98.65) (width 0.381) (layer "F.Cu") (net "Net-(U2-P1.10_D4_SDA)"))
 (via (at 148.416506 98.65) (size 0.6) (drill 0.3) (layers "F.Cu" "B.Cu") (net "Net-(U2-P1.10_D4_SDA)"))
 (segment (start 148.4175 99.04) (end 148.4175 98.851244) (width 0.381) (layer "B.Cu") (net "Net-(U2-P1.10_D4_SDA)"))
 (segment (start 148.4175 98.851244) (end 149.268744 98) (width 0.381) (layer "B.Cu") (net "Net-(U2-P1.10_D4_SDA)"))
 (segment (start 151 94) (end 151.65 93.35) (width 0.381) (layer "F.Cu") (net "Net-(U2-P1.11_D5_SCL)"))
 (segment (start 151.65 93.35) (end 153.918744 93.35) (width 0.381) (layer "F.Cu") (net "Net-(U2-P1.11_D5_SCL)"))
 (via (at 151 94) (size 0.6) (drill 0.3) (layers "F.Cu" "B.Cu") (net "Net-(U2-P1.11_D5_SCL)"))
 (segment (start 148.89 96.11) (end 151 94) (width 0.381) (layer "B.Cu") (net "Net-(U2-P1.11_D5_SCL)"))
 (segment (start 148.416506 96.11) (end 148.89 96.11) (width 0.381) (layer "B.Cu") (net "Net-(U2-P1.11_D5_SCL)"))
 (segment (start 133.85 101) (end 140.986506 101) (width 0.381) (layer "F.Cu") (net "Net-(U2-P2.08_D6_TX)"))
 (segment (start 131.5 98.65) (end 133.85 101) (width 0.381) (layer "F.Cu") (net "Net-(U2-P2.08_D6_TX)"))
 (segment (start 140.986506 101) (end 148.416506 93.57) (width 0.381) (layer "F.Cu") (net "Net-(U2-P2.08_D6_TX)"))
 (via (at 148.416506 93.57) (size 0.6) (drill 0.3) (layers "F.Cu" "B.Cu") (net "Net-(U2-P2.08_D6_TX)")))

